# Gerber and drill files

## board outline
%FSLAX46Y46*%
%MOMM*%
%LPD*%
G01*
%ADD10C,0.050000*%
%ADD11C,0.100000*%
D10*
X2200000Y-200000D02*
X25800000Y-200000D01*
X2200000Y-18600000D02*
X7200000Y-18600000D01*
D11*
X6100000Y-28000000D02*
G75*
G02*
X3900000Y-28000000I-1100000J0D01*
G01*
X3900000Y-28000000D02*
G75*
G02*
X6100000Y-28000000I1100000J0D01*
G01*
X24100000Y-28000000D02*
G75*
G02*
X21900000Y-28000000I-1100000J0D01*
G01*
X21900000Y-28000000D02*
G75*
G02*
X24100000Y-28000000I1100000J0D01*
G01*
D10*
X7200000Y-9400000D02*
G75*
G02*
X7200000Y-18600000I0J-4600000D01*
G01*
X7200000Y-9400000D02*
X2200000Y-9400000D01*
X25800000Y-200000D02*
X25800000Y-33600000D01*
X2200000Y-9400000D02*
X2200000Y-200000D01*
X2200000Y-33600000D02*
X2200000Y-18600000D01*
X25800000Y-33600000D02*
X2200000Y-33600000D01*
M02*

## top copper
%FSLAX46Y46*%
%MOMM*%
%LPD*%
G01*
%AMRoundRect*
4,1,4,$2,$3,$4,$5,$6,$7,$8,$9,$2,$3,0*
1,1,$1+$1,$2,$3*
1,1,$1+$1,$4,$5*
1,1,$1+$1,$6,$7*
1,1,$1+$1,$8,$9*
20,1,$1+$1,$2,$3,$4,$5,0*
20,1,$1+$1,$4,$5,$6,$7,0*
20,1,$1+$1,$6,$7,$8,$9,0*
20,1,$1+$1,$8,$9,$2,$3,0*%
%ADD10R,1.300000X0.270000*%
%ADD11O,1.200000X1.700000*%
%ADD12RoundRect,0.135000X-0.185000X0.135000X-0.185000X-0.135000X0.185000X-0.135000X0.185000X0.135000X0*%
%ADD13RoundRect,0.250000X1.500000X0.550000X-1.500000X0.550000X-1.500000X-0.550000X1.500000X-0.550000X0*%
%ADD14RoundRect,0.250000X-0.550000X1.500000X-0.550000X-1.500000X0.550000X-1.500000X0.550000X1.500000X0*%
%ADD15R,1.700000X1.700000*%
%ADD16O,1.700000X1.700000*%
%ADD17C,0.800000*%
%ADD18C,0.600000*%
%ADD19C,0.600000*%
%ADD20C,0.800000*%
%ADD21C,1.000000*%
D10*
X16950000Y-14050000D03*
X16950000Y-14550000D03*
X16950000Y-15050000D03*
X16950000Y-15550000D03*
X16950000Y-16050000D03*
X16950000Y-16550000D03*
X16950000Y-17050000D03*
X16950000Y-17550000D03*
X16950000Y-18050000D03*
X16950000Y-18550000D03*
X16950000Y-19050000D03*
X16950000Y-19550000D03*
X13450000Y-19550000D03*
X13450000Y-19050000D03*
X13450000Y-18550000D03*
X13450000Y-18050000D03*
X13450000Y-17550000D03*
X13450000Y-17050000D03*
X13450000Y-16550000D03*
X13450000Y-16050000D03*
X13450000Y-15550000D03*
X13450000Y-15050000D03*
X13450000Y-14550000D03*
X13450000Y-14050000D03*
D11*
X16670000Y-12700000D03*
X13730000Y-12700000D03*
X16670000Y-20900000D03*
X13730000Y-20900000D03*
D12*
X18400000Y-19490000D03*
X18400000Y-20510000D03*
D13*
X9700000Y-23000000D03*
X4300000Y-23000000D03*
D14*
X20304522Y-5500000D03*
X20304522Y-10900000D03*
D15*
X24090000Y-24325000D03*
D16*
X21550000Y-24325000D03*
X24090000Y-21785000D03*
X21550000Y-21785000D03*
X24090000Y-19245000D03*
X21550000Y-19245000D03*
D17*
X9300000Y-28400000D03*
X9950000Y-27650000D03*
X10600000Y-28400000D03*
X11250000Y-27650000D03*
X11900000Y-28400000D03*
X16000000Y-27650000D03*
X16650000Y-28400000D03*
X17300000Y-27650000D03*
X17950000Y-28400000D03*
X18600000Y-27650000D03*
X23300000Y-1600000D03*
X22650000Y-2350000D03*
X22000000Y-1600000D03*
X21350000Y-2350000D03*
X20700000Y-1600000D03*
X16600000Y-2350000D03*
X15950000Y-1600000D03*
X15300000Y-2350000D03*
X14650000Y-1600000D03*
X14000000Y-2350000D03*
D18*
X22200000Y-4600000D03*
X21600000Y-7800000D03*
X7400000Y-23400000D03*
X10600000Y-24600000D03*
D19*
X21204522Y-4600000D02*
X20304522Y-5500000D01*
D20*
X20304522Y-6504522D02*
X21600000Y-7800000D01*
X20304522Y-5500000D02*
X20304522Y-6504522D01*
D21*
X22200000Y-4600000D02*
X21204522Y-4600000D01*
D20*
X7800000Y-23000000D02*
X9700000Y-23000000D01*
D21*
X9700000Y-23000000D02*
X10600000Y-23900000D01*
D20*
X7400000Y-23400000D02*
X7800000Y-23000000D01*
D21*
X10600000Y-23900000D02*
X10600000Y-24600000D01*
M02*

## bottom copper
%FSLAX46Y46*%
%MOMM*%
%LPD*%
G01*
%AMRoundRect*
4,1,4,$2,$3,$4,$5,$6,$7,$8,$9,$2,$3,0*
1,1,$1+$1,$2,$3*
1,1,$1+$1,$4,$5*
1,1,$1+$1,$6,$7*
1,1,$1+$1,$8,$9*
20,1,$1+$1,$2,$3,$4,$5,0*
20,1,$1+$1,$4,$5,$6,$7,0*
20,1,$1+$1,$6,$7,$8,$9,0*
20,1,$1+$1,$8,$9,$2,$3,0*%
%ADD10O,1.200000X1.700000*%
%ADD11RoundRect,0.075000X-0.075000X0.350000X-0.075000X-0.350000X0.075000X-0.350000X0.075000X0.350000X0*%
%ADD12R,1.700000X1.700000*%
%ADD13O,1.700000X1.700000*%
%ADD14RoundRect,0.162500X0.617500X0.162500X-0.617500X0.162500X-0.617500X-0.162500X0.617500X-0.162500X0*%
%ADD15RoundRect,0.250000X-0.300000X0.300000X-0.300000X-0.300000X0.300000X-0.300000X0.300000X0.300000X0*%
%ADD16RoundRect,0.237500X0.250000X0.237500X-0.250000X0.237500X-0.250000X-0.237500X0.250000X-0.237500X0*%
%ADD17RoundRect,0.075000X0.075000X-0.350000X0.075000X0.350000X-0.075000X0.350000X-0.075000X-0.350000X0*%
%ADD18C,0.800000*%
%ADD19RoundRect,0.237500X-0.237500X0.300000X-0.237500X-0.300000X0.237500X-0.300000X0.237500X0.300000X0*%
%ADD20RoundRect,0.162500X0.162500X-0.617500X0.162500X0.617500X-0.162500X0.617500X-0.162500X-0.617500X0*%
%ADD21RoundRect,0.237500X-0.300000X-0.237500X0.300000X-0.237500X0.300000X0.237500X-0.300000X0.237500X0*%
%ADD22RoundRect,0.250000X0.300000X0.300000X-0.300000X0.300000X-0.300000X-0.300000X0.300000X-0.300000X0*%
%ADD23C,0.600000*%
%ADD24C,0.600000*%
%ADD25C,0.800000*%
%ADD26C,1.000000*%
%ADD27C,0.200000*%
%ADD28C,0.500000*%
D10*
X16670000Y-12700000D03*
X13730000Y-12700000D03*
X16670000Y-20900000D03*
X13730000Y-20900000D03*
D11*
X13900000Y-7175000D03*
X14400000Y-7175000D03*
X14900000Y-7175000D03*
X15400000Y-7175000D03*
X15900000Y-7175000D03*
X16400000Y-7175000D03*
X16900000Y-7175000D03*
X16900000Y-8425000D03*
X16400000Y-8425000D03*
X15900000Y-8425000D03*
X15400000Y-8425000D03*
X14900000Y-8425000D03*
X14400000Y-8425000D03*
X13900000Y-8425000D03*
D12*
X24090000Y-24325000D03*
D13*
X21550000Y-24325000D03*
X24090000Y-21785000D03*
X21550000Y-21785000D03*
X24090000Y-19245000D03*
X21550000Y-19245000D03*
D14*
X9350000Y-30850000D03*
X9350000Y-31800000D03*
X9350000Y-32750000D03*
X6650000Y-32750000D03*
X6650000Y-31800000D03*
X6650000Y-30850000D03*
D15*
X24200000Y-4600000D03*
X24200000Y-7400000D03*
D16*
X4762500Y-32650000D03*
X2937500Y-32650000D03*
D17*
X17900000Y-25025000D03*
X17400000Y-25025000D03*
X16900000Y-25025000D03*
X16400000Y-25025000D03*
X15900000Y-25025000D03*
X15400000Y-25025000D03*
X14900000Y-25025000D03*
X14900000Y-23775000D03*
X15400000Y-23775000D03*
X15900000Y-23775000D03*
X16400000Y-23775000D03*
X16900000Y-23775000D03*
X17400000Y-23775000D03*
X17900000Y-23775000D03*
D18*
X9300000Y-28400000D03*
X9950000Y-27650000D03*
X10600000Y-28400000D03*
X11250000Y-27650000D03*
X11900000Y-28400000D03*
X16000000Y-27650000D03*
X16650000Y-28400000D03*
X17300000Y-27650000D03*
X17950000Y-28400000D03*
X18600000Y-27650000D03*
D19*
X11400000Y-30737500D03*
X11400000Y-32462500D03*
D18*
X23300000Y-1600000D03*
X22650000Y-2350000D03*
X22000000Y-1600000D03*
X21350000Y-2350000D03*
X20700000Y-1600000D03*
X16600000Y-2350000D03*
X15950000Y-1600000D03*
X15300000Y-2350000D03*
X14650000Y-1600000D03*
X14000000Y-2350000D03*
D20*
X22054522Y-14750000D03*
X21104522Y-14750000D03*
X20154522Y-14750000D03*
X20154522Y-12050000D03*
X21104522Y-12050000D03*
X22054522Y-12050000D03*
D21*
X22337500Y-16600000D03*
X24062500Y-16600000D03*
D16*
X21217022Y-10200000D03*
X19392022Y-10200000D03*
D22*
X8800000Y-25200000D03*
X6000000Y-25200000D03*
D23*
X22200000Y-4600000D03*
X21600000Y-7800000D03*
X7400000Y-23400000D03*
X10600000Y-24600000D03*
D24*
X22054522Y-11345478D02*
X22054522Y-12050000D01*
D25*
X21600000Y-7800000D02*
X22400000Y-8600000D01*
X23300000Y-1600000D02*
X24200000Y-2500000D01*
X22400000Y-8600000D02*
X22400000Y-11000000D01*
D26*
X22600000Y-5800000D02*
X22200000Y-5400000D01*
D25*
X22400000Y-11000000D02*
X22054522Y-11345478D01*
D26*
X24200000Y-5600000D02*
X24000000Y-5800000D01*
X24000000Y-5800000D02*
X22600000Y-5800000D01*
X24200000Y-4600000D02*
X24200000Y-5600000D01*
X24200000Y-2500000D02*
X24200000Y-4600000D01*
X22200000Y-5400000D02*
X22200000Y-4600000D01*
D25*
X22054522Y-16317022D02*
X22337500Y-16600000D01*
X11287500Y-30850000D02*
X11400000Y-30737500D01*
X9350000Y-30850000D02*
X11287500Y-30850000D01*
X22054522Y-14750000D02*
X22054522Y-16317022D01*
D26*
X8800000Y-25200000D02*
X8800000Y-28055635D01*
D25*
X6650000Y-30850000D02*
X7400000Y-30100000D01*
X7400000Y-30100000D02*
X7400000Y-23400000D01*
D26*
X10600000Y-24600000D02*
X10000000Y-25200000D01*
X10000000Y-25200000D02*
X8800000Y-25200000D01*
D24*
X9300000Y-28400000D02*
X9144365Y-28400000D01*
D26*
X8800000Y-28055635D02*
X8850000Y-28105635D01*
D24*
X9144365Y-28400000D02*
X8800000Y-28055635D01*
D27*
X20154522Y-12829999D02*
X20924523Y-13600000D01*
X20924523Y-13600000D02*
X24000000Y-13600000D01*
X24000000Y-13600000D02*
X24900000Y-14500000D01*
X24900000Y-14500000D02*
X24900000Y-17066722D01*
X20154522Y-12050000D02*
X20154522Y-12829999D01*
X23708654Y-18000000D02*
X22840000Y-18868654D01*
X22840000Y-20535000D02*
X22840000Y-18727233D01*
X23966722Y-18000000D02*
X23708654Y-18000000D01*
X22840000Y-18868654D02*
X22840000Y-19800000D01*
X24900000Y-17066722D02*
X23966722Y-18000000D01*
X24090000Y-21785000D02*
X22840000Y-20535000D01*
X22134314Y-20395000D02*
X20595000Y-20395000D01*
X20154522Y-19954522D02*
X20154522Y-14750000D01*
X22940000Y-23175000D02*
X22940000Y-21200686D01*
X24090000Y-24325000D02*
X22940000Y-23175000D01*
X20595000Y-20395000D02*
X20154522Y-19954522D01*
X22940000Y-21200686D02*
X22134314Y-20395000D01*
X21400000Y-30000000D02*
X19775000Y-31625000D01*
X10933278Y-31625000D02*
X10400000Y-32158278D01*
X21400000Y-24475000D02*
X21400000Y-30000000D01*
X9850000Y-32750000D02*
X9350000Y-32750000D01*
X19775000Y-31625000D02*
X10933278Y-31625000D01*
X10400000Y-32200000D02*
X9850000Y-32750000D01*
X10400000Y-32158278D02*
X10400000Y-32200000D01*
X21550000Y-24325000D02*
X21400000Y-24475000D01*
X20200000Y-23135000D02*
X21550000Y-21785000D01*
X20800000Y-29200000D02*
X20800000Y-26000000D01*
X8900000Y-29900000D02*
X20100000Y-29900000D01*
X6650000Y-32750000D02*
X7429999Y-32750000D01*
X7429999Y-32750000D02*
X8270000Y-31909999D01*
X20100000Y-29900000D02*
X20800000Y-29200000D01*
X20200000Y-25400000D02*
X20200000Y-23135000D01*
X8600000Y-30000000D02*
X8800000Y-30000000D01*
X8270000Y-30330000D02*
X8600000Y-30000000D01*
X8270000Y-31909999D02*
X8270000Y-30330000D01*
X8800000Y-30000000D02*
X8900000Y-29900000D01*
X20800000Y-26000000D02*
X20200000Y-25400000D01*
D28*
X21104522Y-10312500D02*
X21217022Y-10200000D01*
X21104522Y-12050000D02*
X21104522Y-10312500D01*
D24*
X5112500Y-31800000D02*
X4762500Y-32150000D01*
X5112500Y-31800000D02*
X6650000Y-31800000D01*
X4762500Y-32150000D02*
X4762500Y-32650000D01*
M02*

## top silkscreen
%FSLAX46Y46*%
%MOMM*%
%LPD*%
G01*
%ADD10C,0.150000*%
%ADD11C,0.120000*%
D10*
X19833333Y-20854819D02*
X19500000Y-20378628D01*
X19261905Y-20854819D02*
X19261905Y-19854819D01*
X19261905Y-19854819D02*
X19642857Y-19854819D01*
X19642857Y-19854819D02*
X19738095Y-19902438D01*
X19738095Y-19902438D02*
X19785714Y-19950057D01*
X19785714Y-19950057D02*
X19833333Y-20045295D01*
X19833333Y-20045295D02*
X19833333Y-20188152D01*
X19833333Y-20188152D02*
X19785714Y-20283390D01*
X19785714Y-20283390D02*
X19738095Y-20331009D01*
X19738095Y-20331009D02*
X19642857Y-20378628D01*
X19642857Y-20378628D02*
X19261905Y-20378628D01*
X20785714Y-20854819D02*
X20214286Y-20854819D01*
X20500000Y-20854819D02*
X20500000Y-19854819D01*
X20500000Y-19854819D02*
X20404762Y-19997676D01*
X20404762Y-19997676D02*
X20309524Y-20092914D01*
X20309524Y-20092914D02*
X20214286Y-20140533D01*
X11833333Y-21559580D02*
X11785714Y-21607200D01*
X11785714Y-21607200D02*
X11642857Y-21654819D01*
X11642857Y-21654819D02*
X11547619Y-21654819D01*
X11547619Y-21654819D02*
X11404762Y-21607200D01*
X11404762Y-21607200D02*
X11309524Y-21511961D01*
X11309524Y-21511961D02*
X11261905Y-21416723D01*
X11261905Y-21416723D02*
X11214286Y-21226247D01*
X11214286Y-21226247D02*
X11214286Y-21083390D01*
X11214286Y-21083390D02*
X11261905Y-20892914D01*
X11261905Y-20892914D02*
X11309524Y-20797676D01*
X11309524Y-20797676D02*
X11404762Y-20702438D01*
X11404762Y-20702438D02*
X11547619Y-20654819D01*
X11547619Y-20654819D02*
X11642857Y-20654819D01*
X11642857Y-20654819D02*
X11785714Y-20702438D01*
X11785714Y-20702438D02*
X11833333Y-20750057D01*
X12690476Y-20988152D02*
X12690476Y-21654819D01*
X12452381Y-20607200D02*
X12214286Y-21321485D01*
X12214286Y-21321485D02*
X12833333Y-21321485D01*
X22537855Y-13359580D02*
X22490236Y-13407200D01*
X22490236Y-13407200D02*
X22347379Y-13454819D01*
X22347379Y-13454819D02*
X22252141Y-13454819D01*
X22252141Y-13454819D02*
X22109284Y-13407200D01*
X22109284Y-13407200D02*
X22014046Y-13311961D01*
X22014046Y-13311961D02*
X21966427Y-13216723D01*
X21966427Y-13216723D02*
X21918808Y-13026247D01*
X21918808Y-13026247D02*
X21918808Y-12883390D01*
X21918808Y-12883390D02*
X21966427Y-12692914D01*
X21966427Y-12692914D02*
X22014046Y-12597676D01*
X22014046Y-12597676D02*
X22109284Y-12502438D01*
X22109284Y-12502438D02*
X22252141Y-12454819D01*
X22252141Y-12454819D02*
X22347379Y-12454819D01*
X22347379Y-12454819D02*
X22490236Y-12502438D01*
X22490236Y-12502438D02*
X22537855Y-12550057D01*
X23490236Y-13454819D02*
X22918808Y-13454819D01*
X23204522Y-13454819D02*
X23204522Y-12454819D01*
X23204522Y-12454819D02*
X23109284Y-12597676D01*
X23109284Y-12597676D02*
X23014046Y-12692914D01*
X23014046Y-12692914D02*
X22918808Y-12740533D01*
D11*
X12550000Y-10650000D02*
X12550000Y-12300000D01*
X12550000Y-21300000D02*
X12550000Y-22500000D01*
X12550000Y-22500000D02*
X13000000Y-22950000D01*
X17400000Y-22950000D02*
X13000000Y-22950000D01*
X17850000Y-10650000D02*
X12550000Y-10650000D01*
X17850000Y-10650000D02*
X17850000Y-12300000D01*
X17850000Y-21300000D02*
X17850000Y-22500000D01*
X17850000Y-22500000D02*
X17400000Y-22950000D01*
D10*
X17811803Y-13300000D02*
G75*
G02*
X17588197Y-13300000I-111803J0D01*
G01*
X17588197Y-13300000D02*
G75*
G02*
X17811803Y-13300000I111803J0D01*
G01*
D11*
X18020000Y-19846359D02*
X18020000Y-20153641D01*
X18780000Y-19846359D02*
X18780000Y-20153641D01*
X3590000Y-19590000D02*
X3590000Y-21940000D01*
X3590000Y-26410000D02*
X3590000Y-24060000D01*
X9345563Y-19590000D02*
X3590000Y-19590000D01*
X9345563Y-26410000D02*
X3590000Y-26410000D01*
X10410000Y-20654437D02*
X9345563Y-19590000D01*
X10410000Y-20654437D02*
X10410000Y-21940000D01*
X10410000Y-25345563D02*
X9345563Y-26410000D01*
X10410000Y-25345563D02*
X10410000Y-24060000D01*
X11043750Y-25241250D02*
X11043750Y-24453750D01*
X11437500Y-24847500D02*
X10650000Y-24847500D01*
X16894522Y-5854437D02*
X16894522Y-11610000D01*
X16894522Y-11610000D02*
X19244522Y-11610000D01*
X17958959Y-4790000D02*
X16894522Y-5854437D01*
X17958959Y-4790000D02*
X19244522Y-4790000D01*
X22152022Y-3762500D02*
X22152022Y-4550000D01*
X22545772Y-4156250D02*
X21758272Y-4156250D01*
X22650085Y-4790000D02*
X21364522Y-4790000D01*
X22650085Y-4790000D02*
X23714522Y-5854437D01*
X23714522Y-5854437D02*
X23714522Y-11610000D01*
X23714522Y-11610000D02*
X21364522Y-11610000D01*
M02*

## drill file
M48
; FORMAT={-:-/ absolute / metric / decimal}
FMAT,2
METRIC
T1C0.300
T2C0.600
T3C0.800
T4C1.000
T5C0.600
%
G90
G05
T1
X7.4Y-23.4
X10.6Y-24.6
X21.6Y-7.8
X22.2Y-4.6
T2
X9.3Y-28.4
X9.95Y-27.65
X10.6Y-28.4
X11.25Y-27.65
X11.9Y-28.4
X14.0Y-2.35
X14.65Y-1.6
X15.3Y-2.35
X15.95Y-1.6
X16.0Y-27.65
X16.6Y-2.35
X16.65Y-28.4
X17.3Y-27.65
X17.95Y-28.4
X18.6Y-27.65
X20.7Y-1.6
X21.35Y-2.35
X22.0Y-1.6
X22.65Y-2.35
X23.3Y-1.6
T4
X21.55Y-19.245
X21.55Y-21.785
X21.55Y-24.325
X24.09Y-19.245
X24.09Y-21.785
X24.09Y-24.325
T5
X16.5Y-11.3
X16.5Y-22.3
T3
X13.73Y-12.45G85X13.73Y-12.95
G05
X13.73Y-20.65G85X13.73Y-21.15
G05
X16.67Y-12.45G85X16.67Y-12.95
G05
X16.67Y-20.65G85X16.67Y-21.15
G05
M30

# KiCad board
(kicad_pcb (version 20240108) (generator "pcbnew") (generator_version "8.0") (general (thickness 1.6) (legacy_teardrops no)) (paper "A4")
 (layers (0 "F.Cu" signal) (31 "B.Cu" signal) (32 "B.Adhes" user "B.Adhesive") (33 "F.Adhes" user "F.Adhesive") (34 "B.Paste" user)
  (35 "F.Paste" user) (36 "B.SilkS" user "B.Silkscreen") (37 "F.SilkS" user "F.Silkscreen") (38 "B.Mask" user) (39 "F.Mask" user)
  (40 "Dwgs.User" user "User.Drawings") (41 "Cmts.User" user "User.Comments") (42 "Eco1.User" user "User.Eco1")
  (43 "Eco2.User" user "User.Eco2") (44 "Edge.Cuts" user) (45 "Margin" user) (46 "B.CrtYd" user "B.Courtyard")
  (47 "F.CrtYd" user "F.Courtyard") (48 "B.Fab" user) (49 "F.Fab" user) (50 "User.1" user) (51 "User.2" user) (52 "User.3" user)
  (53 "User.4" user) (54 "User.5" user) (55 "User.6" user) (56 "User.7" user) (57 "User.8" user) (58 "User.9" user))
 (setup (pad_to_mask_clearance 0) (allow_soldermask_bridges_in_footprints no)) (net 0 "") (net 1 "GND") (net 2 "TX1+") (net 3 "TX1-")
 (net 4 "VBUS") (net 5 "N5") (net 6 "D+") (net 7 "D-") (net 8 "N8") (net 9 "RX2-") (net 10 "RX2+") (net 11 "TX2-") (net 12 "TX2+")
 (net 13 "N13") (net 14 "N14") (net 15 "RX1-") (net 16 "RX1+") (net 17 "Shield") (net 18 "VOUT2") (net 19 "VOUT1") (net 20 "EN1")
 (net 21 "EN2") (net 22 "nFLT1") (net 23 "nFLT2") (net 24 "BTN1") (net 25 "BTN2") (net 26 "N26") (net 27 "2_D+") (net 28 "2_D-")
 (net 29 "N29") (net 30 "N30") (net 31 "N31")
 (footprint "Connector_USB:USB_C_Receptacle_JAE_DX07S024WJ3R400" (layer "F.Cu") (at 15.2 16.8 -90)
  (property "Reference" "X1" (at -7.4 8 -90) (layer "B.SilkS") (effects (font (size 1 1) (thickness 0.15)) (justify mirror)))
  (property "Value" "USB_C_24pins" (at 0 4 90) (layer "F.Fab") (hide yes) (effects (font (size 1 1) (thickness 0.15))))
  (fp_line (start -6.15 2.65) (end -4.5 2.65) (stroke (width 0.12) (type solid)) (layer "F.SilkS"))
  (fp_line (start 4.5 2.65) (end 5.7 2.65) (stroke (width 0.12) (type solid)) (layer "F.SilkS"))
  (fp_line (start 5.7 2.65) (end 6.15 2.2) (stroke (width 0.12) (type solid)) (layer "F.SilkS"))
  (fp_line (start 6.15 -2.2) (end 6.15 2.2) (stroke (width 0.12) (type solid)) (layer "F.SilkS"))
  (fp_line (start -6.15 -2.65) (end -6.15 2.65) (stroke (width 0.12) (type solid)) (layer "F.SilkS"))
  (fp_line (start -6.15 -2.65) (end -4.5 -2.65) (stroke (width 0.12) (type solid)) (layer "F.SilkS"))
  (fp_line (start 4.5 -2.65) (end 5.7 -2.65) (stroke (width 0.12) (type solid)) (layer "F.SilkS"))
  (fp_line (start 5.7 -2.65) (end 6.15 -2.2) (stroke (width 0.12) (type solid)) (layer "F.SilkS"))
  (fp_circle (center -3.5 -2.5) (end -3.388197 -2.5) (stroke (width 0.15) (type solid)) (fill none) (layer "F.SilkS"))
  (pad "" np_thru_hole circle (at -5.5 -1.3 270) (size 0.6 0.6) (drill 0.6) (layers "*.Cu" "*.Mask"))
  (pad "" np_thru_hole circle (at 5.5 -1.3 270) (size 0.6 0.6) (drill 0.6) (layers "*.Cu" "*.Mask"))
  (pad "A1" smd rect (at -2.75 -1.75 270) (size 0.27 1.3) (layers "F.Cu" "F.Paste" "F.Mask") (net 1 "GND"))
  (pad "A2" smd rect (at -2.25 -1.75 270) (size 0.27 1.3) (layers "F.Cu" "F.Paste" "F.Mask") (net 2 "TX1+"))
  (pad "A3" smd rect (at -1.75 -1.75 270) (size 0.27 1.3) (layers "F.Cu" "F.Paste" "F.Mask") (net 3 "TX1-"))
  (pad "A4" smd rect (at -1.25 -1.75 270) (size 0.27 1.3) (layers "F.Cu" "F.Paste" "F.Mask") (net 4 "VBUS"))
  (pad "A5" smd rect (at -0.75 -1.75 270) (size 0.27 1.3) (layers "F.Cu" "F.Paste" "F.Mask") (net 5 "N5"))
  (pad "A6" smd rect (at -0.25 -1.75 270) (size 0.27 1.3) (layers "F.Cu" "F.Paste" "F.Mask") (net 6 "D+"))
  (pad "A7" smd rect (at 0.25 -1.75 270) (size 0.27 1.3) (layers "F.Cu" "F.Paste" "F.Mask") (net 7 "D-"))
  (pad "A8" smd rect (at 0.75 -1.75 270) (size 0.27 1.3) (layers "F.Cu" "F.Paste" "F.Mask") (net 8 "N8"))
  (pad "A9" smd rect (at 1.25 -1.75 270) (size 0.27 1.3) (layers "F.Cu" "F.Paste" "F.Mask") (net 4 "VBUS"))
  (pad "A10" smd rect (at 1.75 -1.75 270) (size 0.27 1.3) (layers "F.Cu" "F.Paste" "F.Mask") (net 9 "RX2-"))
  (pad "A11" smd rect (at 2.25 -1.75 270) (size 0.27 1.3) (layers "F.Cu" "F.Paste" "F.Mask") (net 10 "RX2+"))
  (pad "A12" smd rect (at 2.75 -1.75 270) (size 0.27 1.3) (layers "F.Cu" "F.Paste" "F.Mask") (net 1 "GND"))
  (pad "B1" smd rect (at 2.75 1.75 270) (size 0.27 1.3) (layers "F.Cu" "F.Paste" "F.Mask") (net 1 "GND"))
  (pad "B2" smd rect (at 2.25 1.75 270) (size 0.27 1.3) (layers "F.Cu" "F.Paste" "F.Mask") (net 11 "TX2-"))
  (pad "B3" smd rect (at 1.75 1.75 270) (size 0.27 1.3) (layers "F.Cu" "F.Paste" "F.Mask") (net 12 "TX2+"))
  (pad "B4" smd rect (at 1.25 1.75 270) (size 0.27 1.3) (layers "F.Cu" "F.Paste" "F.Mask") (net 4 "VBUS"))
  (pad "B5" smd rect (at 0.75 1.75 270) (size 0.27 1.3) (layers "F.Cu" "F.Paste" "F.Mask") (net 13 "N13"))
  (pad "B6" smd rect (at 0.25 1.75 270) (size 0.27 1.3) (layers "F.Cu" "F.Paste" "F.Mask") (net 6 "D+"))
  (pad "B7" smd rect (at -0.25 1.75 270) (size 0.27 1.3) (layers "F.Cu" "F.Paste" "F.Mask") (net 7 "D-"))
  (pad "B8" smd rect (at -0.75 1.75 270) (size 0.27 1.3) (layers "F.Cu" "F.Paste" "F.Mask") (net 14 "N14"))
  (pad "B9" smd rect (at -1.25 1.75 270) (size 0.27 1.3) (layers "F.Cu" "F.Paste" "F.Mask") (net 4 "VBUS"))
  (pad "B10" smd rect (at -1.75 1.75 270) (size 0.27 1.3) (layers "F.Cu" "F.Paste" "F.Mask") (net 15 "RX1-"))
  (pad "B11" smd rect (at -2.25 1.75 270) (size 0.27 1.3) (layers "F.Cu" "F.Paste" "F.Mask") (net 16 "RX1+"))
  (pad "B12" smd rect (at -2.75 1.75 270) (size 0.27 1.3) (layers "F.Cu" "F.Paste" "F.Mask") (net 1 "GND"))
  (pad "S1" thru_hole oval (at -4.1 -1.47) (size 1.2 1.7) (drill oval 0.8 1.3) (layers "*.Cu" "*.Mask") (remove_unused_layers no)
   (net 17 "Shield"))
  (pad "S1" thru_hole oval (at -4.1 1.47) (size 1.2 1.7) (drill oval 0.8 1.3) (layers "*.Cu" "*.Mask") (remove_unused_layers no)
   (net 17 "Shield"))
  (pad "S1" thru_hole oval (at 4.1 -1.47) (size 1.2 1.7) (drill oval 0.8 1.3) (layers "*.Cu" "*.Mask") (remove_unused_layers no)
   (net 17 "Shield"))
  (pad "S1" thru_hole oval (at 4.1 1.47) (size 1.2 1.7) (drill oval 0.8 1.3) (layers "*.Cu" "*.Mask") (remove_unused_layers no)
   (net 17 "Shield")))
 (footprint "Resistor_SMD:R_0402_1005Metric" (layer "F.Cu") (at 18.4 20 -90)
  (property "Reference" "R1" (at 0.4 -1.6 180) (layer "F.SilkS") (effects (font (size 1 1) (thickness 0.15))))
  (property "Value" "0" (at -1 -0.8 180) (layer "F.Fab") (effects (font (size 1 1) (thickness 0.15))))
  (fp_line (start -0.153641 0.38) (end 0.153641 0.38) (stroke (width 0.12) (type solid)) (layer "F.SilkS"))
  (fp_line (start -0.153641 -0.38) (end 0.153641 -0.38) (stroke (width 0.12) (type solid)) (layer "F.SilkS"))
  (pad "1" smd roundrect (at -0.51 0 270) (size 0.54 0.64) (layers "F.Cu" "F.Paste" "F.Mask") (roundrect_rratio 0.25) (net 17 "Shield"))
  (pad "2" smd roundrect (at 0.51 0 270) (size 0.54 0.64) (layers "F.Cu" "F.Paste" "F.Mask") (roundrect_rratio 0.25) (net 1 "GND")))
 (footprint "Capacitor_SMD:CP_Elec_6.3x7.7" (layer "F.Cu") (at 7 23 180)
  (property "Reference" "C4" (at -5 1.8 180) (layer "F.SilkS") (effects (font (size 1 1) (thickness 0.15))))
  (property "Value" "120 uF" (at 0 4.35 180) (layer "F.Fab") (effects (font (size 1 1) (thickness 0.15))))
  (fp_line (start 3.41 3.41) (end 3.41 1.06) (stroke (width 0.12) (type solid)) (layer "F.SilkS"))
  (fp_line (start 3.41 -3.41) (end 3.41 -1.06) (stroke (width 0.12) (type solid)) (layer "F.SilkS"))
  (fp_line (start -2.345563 3.41) (end 3.41 3.41) (stroke (width 0.12) (type solid)) (layer "F.SilkS"))
  (fp_line (start -2.345563 -3.41) (end 3.41 -3.41) (stroke (width 0.12) (type solid)) (layer "F.SilkS"))
  (fp_line (start -3.41 2.345563) (end -2.345563 3.41) (stroke (width 0.12) (type solid)) (layer "F.SilkS"))
  (fp_line (start -3.41 2.345563) (end -3.41 1.06) (stroke (width 0.12) (type solid)) (layer "F.SilkS"))
  (fp_line (start -3.41 -2.345563) (end -2.345563 -3.41) (stroke (width 0.12) (type solid)) (layer "F.SilkS"))
  (fp_line (start -3.41 -2.345563) (end -3.41 -1.06) (stroke (width 0.12) (type solid)) (layer "F.SilkS"))
  (fp_line (start -4.04375 -2.24125) (end -4.04375 -1.45375) (stroke (width 0.12) (type solid)) (layer "F.SilkS"))
  (fp_line (start -4.4375 -1.8475) (end -3.65 -1.8475) (stroke (width 0.12) (type solid)) (layer "F.SilkS"))
  (pad "1" smd roundrect (at -2.7 0 180) (size 3.5 1.6) (layers "F.Cu" "F.Paste" "F.Mask") (roundrect_rratio 0.15625) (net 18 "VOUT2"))
  (pad "2" smd roundrect (at 2.7 0 180) (size 3.5 1.6) (layers "F.Cu" "F.Paste" "F.Mask") (roundrect_rratio 0.15625) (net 1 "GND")))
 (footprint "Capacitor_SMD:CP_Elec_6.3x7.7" (layer "F.Cu") (at 20.304522 8.2 -90)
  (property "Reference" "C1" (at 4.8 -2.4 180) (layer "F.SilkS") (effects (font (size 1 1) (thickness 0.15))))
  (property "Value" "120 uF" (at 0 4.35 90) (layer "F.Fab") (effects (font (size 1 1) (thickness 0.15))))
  (fp_line (start -2.345563 3.41) (end 3.41 3.41) (stroke (width 0.12) (type solid)) (layer "F.SilkS"))
  (fp_line (start 3.41 3.41) (end 3.41 1.06) (stroke (width 0.12) (type solid)) (layer "F.SilkS"))
  (fp_line (start -3.41 2.345563) (end -2.345563 3.41) (stroke (width 0.12) (type solid)) (layer "F.SilkS"))
  (fp_line (start -3.41 2.345563) (end -3.41 1.06) (stroke (width 0.12) (type solid)) (layer "F.SilkS"))
  (fp_line (start -4.4375 -1.8475) (end -3.65 -1.8475) (stroke (width 0.12) (type solid)) (layer "F.SilkS"))
  (fp_line (start -4.04375 -2.24125) (end -4.04375 -1.45375) (stroke (width 0.12) (type solid)) (layer "F.SilkS"))
  (fp_line (start -3.41 -2.345563) (end -3.41 -1.06) (stroke (width 0.12) (type solid)) (layer "F.SilkS"))
  (fp_line (start -3.41 -2.345563) (end -2.345563 -3.41) (stroke (width 0.12) (type solid)) (layer "F.SilkS"))
  (fp_line (start -2.345563 -3.41) (end 3.41 -3.41) (stroke (width 0.12) (type solid)) (layer "F.SilkS"))
  (fp_line (start 3.41 -3.41) (end 3.41 -1.06) (stroke (width 0.12) (type solid)) (layer "F.SilkS"))
  (pad "1" smd roundrect (at -2.7 0 270) (size 3.5 1.6) (layers "F.Cu" "F.Paste" "F.Mask") (roundrect_rratio 0.15625) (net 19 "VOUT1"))
  (pad "2" smd roundrect (at 2.7 0 270) (size 3.5 1.6) (layers "F.Cu" "F.Paste" "F.Mask") (roundrect_rratio 0.15625) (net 1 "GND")))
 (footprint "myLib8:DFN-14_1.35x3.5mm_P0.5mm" (layer "B.Cu") (at 15.4 7.8 -90)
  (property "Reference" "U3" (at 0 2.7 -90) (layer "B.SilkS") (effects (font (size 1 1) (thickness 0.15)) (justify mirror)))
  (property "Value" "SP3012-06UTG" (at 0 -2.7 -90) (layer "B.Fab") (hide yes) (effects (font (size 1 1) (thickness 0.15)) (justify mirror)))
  (pad "1" smd roundrect (at -0.625 1.5 270) (size 0.85 0.3) (layers "B.Cu" "B.Paste" "B.Mask") (roundrect_rratio 0.25) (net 16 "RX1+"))
  (pad "2" smd roundrect (at -0.625 1 270) (size 0.85 0.3) (layers "B.Cu" "B.Paste" "B.Mask") (roundrect_rratio 0.25) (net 15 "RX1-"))
  (pad "3" smd roundrect (at -0.625 0.5 270) (size 0.85 0.3) (layers "B.Cu" "B.Paste" "B.Mask") (roundrect_rratio 0.25) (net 2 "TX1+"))
  (pad "4" smd roundrect (at -0.625 0 270) (size 0.85 0.3) (layers "B.Cu" "B.Paste" "B.Mask") (roundrect_rratio 0.25) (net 3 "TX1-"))
  (pad "5" smd roundrect (at -0.625 -0.5 270) (size 0.85 0.3) (layers "B.Cu" "B.Paste" "B.Mask") (roundrect_rratio 0.25) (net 1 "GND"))
  (pad "6" smd roundrect (at -0.625 -1 270) (size 0.85 0.3) (layers "B.Cu" "B.Paste" "B.Mask") (roundrect_rratio 0.25) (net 6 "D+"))
  (pad "7" smd roundrect (at -0.625 -1.5 270) (size 0.85 0.3) (layers "B.Cu" "B.Paste" "B.Mask") (roundrect_rratio 0.25) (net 7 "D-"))
  (pad "8" smd roundrect (at 0.625 -1.5 270) (size 0.85 0.3) (layers "B.Cu" "B.Paste" "B.Mask") (roundrect_rratio 0.25) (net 7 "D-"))
  (pad "9" smd roundrect (at 0.625 -1 270) (size 0.85 0.3) (layers "B.Cu" "B.Paste" "B.Mask") (roundrect_rratio 0.25) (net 6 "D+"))
  (pad "10" smd roundrect (at 0.625 -0.5 270) (size 0.85 0.3) (layers "B.Cu" "B.Paste" "B.Mask") (roundrect_rratio 0.25) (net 1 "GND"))
  (pad "11" smd roundrect (at 0.625 0 270) (size 0.85 0.3) (layers "B.Cu" "B.Paste" "B.Mask") (roundrect_rratio 0.25) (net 3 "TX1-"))
  (pad "12" smd roundrect (at 0.625 0.5 270) (size 0.85 0.3) (layers "B.Cu" "B.Paste" "B.Mask") (roundrect_rratio 0.25) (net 2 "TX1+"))
  (pad "13" smd roundrect (at 0.625 1 270) (size 0.85 0.3) (layers "B.Cu" "B.Paste" "B.Mask") (roundrect_rratio 0.25) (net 15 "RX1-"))
  (pad "14" smd roundrect (at 0.625 1.5 270) (size 0.85 0.3) (layers "B.Cu" "B.Paste" "B.Mask") (roundrect_rratio 0.25) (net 16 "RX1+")))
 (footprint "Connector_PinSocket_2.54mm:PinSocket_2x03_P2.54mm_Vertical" (layer "B.Cu") (at 24.09 24.325)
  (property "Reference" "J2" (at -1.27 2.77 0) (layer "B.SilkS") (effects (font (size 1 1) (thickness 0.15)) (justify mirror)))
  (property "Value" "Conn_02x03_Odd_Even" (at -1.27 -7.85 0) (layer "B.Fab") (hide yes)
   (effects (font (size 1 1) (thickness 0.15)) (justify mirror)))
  (pad "1" thru_hole rect (at 0 0) (size 1.7 1.7) (drill 1) (layers "*.Cu" "*.Mask") (remove_unused_layers no) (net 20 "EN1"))
  (pad "2" thru_hole oval (at -2.54 0) (size 1.7 1.7) (drill 1) (layers "*.Cu" "*.Mask") (remove_unused_layers no) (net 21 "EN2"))
  (pad "3" thru_hole oval (at 0 -2.54) (size 1.7 1.7) (drill 1) (layers "*.Cu" "*.Mask") (remove_unused_layers no) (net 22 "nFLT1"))
  (pad "4" thru_hole oval (at -2.54 -2.54) (size 1.7 1.7) (drill 1) (layers "*.Cu" "*.Mask") (remove_unused_layers no) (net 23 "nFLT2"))
  (pad "5" thru_hole oval (at 0 -5.08) (size 1.7 1.7) (drill 1) (layers "*.Cu" "*.Mask") (remove_unused_layers no) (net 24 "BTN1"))
  (pad "6" thru_hole oval (at -2.54 -5.08) (size 1.7 1.7) (drill 1) (layers "*.Cu" "*.Mask") (remove_unused_layers no) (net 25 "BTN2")))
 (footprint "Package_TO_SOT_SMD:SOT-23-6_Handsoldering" (layer "B.Cu") (at 8 31.8 180)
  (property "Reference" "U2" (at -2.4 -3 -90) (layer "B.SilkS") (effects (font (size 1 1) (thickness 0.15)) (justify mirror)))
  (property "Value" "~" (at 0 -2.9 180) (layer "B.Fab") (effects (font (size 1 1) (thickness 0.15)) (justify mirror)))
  (pad "1" smd roundrect (at -1.35 0.95 180) (size 1.56 0.65) (layers "B.Cu" "B.Paste" "B.Mask") (roundrect_rratio 0.25) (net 4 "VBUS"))
  (pad "2" smd roundrect (at -1.35 0 180) (size 1.56 0.65) (layers "B.Cu" "B.Paste" "B.Mask") (roundrect_rratio 0.25) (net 1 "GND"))
  (pad "3" smd roundrect (at -1.35 -0.95 180) (size 1.56 0.65) (layers "B.Cu" "B.Paste" "B.Mask") (roundrect_rratio 0.25) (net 21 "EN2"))
  (pad "4" smd roundrect (at 1.35 -0.95 180) (size 1.56 0.65) (layers "B.Cu" "B.Paste" "B.Mask") (roundrect_rratio 0.25) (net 23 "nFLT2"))
  (pad "5" smd roundrect (at 1.35 0 180) (size 1.56 0.65) (layers "B.Cu" "B.Paste" "B.Mask") (roundrect_rratio 0.25) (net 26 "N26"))
  (pad "6" smd roundrect (at 1.35 0.95 180) (size 1.56 0.65) (layers "B.Cu" "B.Paste" "B.Mask") (roundrect_rratio 0.25) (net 18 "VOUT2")))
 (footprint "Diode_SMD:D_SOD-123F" (layer "B.Cu") (at 24.2 6 -90)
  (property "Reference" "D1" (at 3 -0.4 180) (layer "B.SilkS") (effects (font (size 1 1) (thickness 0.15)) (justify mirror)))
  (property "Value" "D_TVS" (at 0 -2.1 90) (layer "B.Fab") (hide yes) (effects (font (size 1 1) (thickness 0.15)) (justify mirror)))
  (pad "1" smd roundrect (at -1.4 0 270) (size 1.1 1.1) (layers "B.Cu" "B.Paste" "B.Mask") (roundrect_rratio 0.2272727273) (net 19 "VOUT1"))
  (pad "2" smd roundrect (at 1.4 0 270) (size 1.1 1.1) (layers "B.Cu" "B.Paste" "B.Mask") (roundrect_rratio 0.2272727273) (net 1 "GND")))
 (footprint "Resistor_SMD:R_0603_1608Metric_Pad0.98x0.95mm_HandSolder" (layer "B.Cu") (at 3.85 32.65 180)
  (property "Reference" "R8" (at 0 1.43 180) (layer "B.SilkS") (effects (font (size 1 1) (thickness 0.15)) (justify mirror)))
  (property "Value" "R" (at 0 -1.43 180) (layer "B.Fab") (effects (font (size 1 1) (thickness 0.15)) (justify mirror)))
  (pad "1" smd roundrect (at -0.9125 0 180) (size 0.975 0.95) (layers "B.Cu" "B.Paste" "B.Mask") (roundrect_rratio 0.25) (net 26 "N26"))
  (pad "2" smd roundrect (at 0.9125 0 180) (size 0.975 0.95) (layers "B.Cu" "B.Paste" "B.Mask") (roundrect_rratio 0.25) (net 1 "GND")))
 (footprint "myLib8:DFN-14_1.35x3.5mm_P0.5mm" (layer "B.Cu") (at 16.4 24.4 90)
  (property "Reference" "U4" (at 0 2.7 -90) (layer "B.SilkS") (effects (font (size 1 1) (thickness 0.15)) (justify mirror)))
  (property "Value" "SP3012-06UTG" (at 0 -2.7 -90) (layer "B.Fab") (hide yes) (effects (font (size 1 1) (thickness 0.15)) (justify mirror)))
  (pad "1" smd roundrect (at -0.625 1.5 90) (size 0.85 0.3) (layers "B.Cu" "B.Paste" "B.Mask") (roundrect_rratio 0.25) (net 10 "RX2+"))
  (pad "2" smd roundrect (at -0.625 1 90) (size 0.85 0.3) (layers "B.Cu" "B.Paste" "B.Mask") (roundrect_rratio 0.25) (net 9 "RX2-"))
  (pad "3" smd roundrect (at -0.625 0.5 90) (size 0.85 0.3) (layers "B.Cu" "B.Paste" "B.Mask") (roundrect_rratio 0.25) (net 11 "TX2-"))
  (pad "4" smd roundrect (at -0.625 0 90) (size 0.85 0.3) (layers "B.Cu" "B.Paste" "B.Mask") (roundrect_rratio 0.25) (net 12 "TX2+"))
  (pad "5" smd roundrect (at -0.625 -0.5 90) (size 0.85 0.3) (layers "B.Cu" "B.Paste" "B.Mask") (roundrect_rratio 0.25) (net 1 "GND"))
  (pad "6" smd roundrect (at -0.625 -1 90) (size 0.85 0.3) (layers "B.Cu" "B.Paste" "B.Mask") (roundrect_rratio 0.25) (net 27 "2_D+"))
  (pad "7" smd roundrect (at -0.625 -1.5 90) (size 0.85 0.3) (layers "B.Cu" "B.Paste" "B.Mask") (roundrect_rratio 0.25) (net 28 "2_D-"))
  (pad "8" smd roundrect (at 0.625 -1.5 90) (size 0.85 0.3) (layers "B.Cu" "B.Paste" "B.Mask") (roundrect_rratio 0.25) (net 28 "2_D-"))
  (pad "9" smd roundrect (at 0.625 -1 90) (size 0.85 0.3) (layers "B.Cu" "B.Paste" "B.Mask") (roundrect_rratio 0.25) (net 27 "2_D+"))
  (pad "10" smd roundrect (at 0.625 -0.5 90) (size 0.85 0.3) (layers "B.Cu" "B.Paste" "B.Mask") (roundrect_rratio 0.25) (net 1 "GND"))
  (pad "11" smd roundrect (at 0.625 0 90) (size 0.85 0.3) (layers "B.Cu" "B.Paste" "B.Mask") (roundrect_rratio 0.25) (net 12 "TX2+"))
  (pad "12" smd roundrect (at 0.625 0.5 90) (size 0.85 0.3) (layers "B.Cu" "B.Paste" "B.Mask") (roundrect_rratio 0.25) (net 11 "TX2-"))
  (pad "13" smd roundrect (at 0.625 1 90) (size 0.85 0.3) (layers "B.Cu" "B.Paste" "B.Mask") (roundrect_rratio 0.25) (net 9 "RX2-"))
  (pad "14" smd roundrect (at 0.625 1.5 90) (size 0.85 0.3) (layers "B.Cu" "B.Paste" "B.Mask") (roundrect_rratio 0.25) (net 10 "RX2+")))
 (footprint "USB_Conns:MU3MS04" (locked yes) (layer "B.Cu") (at 9.3 28.4 180)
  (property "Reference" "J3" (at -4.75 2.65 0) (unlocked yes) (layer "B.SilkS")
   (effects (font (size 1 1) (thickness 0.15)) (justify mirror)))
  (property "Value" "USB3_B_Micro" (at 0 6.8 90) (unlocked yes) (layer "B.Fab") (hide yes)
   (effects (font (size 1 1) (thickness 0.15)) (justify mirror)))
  (pad "1" thru_hole circle (at 0 0 180) (size 0.8 0.8) (drill 0.6) (layers "*.Cu" "*.Mask") (remove_unused_layers no) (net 18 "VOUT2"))
  (pad "2" thru_hole circle (at -0.65 0.75 180) (size 0.8 0.8) (drill 0.6) (layers "*.Cu" "*.Mask") (remove_unused_layers no)
   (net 28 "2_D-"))
  (pad "3" thru_hole circle (at -1.3 0 180) (size 0.8 0.8) (drill 0.6) (layers "*.Cu" "*.Mask") (remove_unused_layers no) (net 27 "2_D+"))
  (pad "4" thru_hole circle (at -1.95 0.75 180) (size 0.8 0.8) (drill 0.6) (layers "*.Cu" "*.Mask") (remove_unused_layers no) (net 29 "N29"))
  (pad "5" thru_hole circle (at -2.6 0 180) (size 0.8 0.8) (drill 0.6) (layers "*.Cu" "*.Mask") (remove_unused_layers no) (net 1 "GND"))
  (pad "6" thru_hole circle (at -6.7 0.75 180) (size 0.8 0.8) (drill 0.6) (layers "*.Cu" "*.Mask") (remove_unused_layers no) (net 12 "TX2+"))
  (pad "7" thru_hole circle (at -7.35 0 180) (size 0.8 0.8) (drill 0.6) (layers "*.Cu" "*.Mask") (remove_unused_layers no) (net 11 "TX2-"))
  (pad "8" thru_hole circle (at -8 0.75 180) (size 0.8 0.8) (drill 0.6) (layers "*.Cu" "*.Mask") (remove_unused_layers no) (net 1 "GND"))
  (pad "9" thru_hole circle (at -8.65 0 180) (size 0.8 0.8) (drill 0.6) (layers "*.Cu" "*.Mask") (remove_unused_layers no) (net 9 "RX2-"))
  (pad "10" thru_hole circle (at -9.3 0.75 180) (size 0.8 0.8) (drill 0.6) (layers "*.Cu" "*.Mask") (remove_unused_layers no)
   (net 10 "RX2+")))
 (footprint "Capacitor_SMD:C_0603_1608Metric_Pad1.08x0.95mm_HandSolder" (layer "B.Cu") (at 11.4 31.6 -90)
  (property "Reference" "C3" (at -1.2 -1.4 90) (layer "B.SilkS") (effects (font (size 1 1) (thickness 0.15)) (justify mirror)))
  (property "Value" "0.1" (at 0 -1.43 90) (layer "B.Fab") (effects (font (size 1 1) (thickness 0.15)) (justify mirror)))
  (pad "1" smd roundrect (at -0.8625 0 270) (size 1.075 0.95) (layers "B.Cu" "B.Paste" "B.Mask") (roundrect_rratio 0.25) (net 4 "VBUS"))
  (pad "2" smd roundrect (at 0.8625 0 270) (size 1.075 0.95) (layers "B.Cu" "B.Paste" "B.Mask") (roundrect_rratio 0.25) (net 1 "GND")))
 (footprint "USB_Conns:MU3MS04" (layer "B.Cu") (at 23.3 1.6)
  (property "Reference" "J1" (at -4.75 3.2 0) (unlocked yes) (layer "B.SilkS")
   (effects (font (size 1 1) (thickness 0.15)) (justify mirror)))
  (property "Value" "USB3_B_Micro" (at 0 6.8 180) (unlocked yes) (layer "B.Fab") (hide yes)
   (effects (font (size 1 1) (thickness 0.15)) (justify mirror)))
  (pad "1" thru_hole circle (at 0 0) (size 0.8 0.8) (drill 0.6) (layers "*.Cu" "*.Mask") (remove_unused_layers no) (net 19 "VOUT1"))
  (pad "2" thru_hole circle (at -0.65 0.75) (size 0.8 0.8) (drill 0.6) (layers "*.Cu" "*.Mask") (remove_unused_layers no) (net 7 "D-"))
  (pad "3" thru_hole circle (at -1.3 0) (size 0.8 0.8) (drill 0.6) (layers "*.Cu" "*.Mask") (remove_unused_layers no) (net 6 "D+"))
  (pad "4" thru_hole circle (at -1.95 0.75) (size 0.8 0.8) (drill 0.6) (layers "*.Cu" "*.Mask") (remove_unused_layers no) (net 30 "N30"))
  (pad "5" thru_hole circle (at -2.6 0) (size 0.8 0.8) (drill 0.6) (layers "*.Cu" "*.Mask") (remove_unused_layers no) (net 1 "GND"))
  (pad "6" thru_hole circle (at -6.7 0.75) (size 0.8 0.8) (drill 0.6) (layers "*.Cu" "*.Mask") (remove_unused_layers no) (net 3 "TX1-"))
  (pad "7" thru_hole circle (at -7.35 0) (size 0.8 0.8) (drill 0.6) (layers "*.Cu" "*.Mask") (remove_unused_layers no) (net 2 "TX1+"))
  (pad "8" thru_hole circle (at -8 0.75) (size 0.8 0.8) (drill 0.6) (layers "*.Cu" "*.Mask") (remove_unused_layers no) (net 1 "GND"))
  (pad "9" thru_hole circle (at -8.65 0) (size 0.8 0.8) (drill 0.6) (layers "*.Cu" "*.Mask") (remove_unused_layers no) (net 15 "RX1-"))
  (pad "10" thru_hole circle (at -9.3 0.75) (size 0.8 0.8) (drill 0.6) (layers "*.Cu" "*.Mask") (remove_unused_layers no) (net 16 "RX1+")))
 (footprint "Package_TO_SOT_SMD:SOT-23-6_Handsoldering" (layer "B.Cu") (at 21.104522 13.4 90)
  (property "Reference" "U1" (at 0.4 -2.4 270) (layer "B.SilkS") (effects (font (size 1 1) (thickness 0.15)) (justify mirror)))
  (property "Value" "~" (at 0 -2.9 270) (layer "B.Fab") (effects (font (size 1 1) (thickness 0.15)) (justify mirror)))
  (pad "1" smd roundrect (at -1.35 0.95 90) (size 1.56 0.65) (layers "B.Cu" "B.Paste" "B.Mask") (roundrect_rratio 0.25) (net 4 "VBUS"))
  (pad "2" smd roundrect (at -1.35 0 90) (size 1.56 0.65) (layers "B.Cu" "B.Paste" "B.Mask") (roundrect_rratio 0.25) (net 1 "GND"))
  (pad "3" smd roundrect (at -1.35 -0.95 90) (size 1.56 0.65) (layers "B.Cu" "B.Paste" "B.Mask") (roundrect_rratio 0.25) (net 20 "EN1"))
  (pad "4" smd roundrect (at 1.35 -0.95 90) (size 1.56 0.65) (layers "B.Cu" "B.Paste" "B.Mask") (roundrect_rratio 0.25) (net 22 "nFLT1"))
  (pad "5" smd roundrect (at 1.35 0 90) (size 1.56 0.65) (layers "B.Cu" "B.Paste" "B.Mask") (roundrect_rratio 0.25) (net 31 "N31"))
  (pad "6" smd roundrect (at 1.35 0.95 90) (size 1.56 0.65) (layers "B.Cu" "B.Paste" "B.Mask") (roundrect_rratio 0.25) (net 19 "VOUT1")))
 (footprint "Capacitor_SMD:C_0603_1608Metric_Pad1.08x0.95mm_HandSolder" (layer "B.Cu") (at 23.2 16.6)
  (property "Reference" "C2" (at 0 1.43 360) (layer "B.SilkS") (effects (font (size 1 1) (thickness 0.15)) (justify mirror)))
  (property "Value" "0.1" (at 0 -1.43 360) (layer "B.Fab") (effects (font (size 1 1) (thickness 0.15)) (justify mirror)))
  (pad "1" smd roundrect (at -0.8625 0) (size 1.075 0.95) (layers "B.Cu" "B.Paste" "B.Mask") (roundrect_rratio 0.25) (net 4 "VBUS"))
  (pad "2" smd roundrect (at 0.8625 0) (size 1.075 0.95) (layers "B.Cu" "B.Paste" "B.Mask") (roundrect_rratio 0.25) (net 1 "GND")))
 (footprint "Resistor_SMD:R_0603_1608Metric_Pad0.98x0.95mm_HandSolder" (layer "B.Cu") (at 20.304522 10.2 180)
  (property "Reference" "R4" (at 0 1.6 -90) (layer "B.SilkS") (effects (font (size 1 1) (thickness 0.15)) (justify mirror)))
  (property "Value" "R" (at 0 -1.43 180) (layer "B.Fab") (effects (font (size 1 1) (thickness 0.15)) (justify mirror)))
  (pad "1" smd roundrect (at -0.9125 0 180) (size 0.975 0.95) (layers "B.Cu" "B.Paste" "B.Mask") (roundrect_rratio 0.25) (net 31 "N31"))
  (pad "2" smd roundrect (at 0.9125 0 180) (size 0.975 0.95) (layers "B.Cu" "B.Paste" "B.Mask") (roundrect_rratio 0.25) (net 1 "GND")))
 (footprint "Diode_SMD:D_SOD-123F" (layer "B.Cu") (at 7.4 25.2 180)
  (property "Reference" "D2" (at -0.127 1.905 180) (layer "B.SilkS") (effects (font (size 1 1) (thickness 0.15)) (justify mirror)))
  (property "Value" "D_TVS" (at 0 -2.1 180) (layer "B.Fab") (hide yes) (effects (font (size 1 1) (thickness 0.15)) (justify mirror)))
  (pad "1" smd roundrect (at -1.4 0 180) (size 1.1 1.1) (layers "B.Cu" "B.Paste" "B.Mask") (roundrect_rratio 0.2272727273) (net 18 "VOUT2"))
  (pad "2" smd roundrect (at 1.4 0 180) (size 1.1 1.1) (layers "B.Cu" "B.Paste" "B.Mask") (roundrect_rratio 0.2272727273) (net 1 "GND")))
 (gr_line (start 2.2 0.2) (end 25.8 0.2) (locked yes) (stroke (width 0.05) (type default)) (layer "Edge.Cuts"))
 (gr_line (start 2.2 18.6) (end 7.2 18.6) (locked yes) (stroke (width 0.05) (type default)) (layer "Edge.Cuts"))
 (gr_circle (center 5 28) (end 6.1 28) (locked yes) (stroke (width 0.1) (type default)) (fill none) (layer "Edge.Cuts"))
 (gr_circle (center 23 28) (end 24.1 28) (locked yes) (stroke (width 0.1) (type default)) (fill none) (layer "Edge.Cuts"))
 (gr_arc (start 7.2 9.4) (mid 11.8 14) (end 7.2 18.6) (locked yes) (stroke (width 0.05) (type default)) (layer "Edge.Cuts"))
 (gr_line (start 7.2 9.4) (end 2.2 9.4) (locked yes) (stroke (width 0.05) (type default)) (layer "Edge.Cuts"))
 (gr_line (start 25.8 0.2) (end 25.8 33.6) (locked yes) (stroke (width 0.05) (type default)) (layer "Edge.Cuts"))
 (gr_line (start 2.2 9.4) (end 2.2 0.2) (locked yes) (stroke (width 0.05) (type default)) (layer "Edge.Cuts"))
 (gr_line (start 2.2 33.6) (end 2.2 18.6) (locked yes) (stroke (width 0.05) (type default)) (layer "Edge.Cuts"))
 (gr_line (start 25.8 33.6) (end 2.2 33.6) (locked yes) (stroke (width 0.05) (type default)) (layer "Edge.Cuts"))
 (segment (start 21.204522 4.6) (end 20.304522 5.5) (width 0.6) (layer "F.Cu") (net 19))
 (segment (start 20.304522 6.504522) (end 21.6 7.8) (width 0.8) (layer "F.Cu") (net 19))
 (segment (start 20.304522 5.5) (end 20.304522 6.504522) (width 0.8) (layer "F.Cu") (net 19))
 (segment (start 22.2 4.6) (end 21.204522 4.6) (width 1) (layer "F.Cu") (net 19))
 (via (at 22.2 4.6) (size 0.6) (drill 0.3) (layers "F.Cu" "B.Cu") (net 19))
 (via (at 21.6 7.8) (size 0.6) (drill 0.3) (layers "F.Cu" "B.Cu") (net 19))
 (segment (start 22.054522 11.345478) (end 22.054522 12.05) (width 0.6) (layer "B.Cu") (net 19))
 (segment (start 21.6 7.8) (end 22.4 8.6) (width 0.8) (layer "B.Cu") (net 19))
 (segment (start 23.3 1.6) (end 24.2 2.5) (width 0.8) (layer "B.Cu") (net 19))
 (segment (start 22.4 8.6) (end 22.4 11) (width 0.8) (layer "B.Cu") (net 19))
 (segment (start 22.6 5.8) (end 22.2 5.4) (width 1) (layer "B.Cu") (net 19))
 (segment (start 22.4 11) (end 22.054522 11.345478) (width 0.8) (layer "B.Cu") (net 19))
 (segment (start 24.2 5.6) (end 24 5.8) (width 1) (layer "B.Cu") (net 19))
 (segment (start 24 5.8) (end 22.6 5.8) (width 1) (layer "B.Cu") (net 19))
 (segment (start 24.2 4.6) (end 24.2 5.6) (width 1) (layer "B.Cu") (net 19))
 (segment (start 24.2 2.5) (end 24.2 4.6) (width 1) (layer "B.Cu") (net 19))
 (segment (start 22.2 5.4) (end 22.2 4.6) (width 1) (layer "B.Cu") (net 19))
 (segment (start 22.054522 16.317022) (end 22.3375 16.6) (width 0.8) (layer "B.Cu") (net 4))
 (segment (start 11.2875 30.85) (end 11.4 30.7375) (width 0.8) (layer "B.Cu") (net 4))
 (segment (start 9.35 30.85) (end 11.2875 30.85) (width 0.8) (layer "B.Cu") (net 4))
 (segment (start 22.054522 14.75) (end 22.054522 16.317022) (width 0.8) (layer "B.Cu") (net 4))
 (segment (start 7.8 23) (end 9.7 23) (width 0.8) (layer "F.Cu") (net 18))
 (segment (start 9.7 23) (end 10.6 23.9) (width 1) (layer "F.Cu") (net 18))
 (segment (start 7.4 23.4) (end 7.8 23) (width 0.8) (layer "F.Cu") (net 18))
 (segment (start 10.6 23.9) (end 10.6 24.6) (width 1) (layer "F.Cu") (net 18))
 (via (at 7.4 23.4) (size 0.6) (drill 0.3) (layers "F.Cu" "B.Cu") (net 18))
 (via (at 10.6 24.6) (size 0.6) (drill 0.3) (layers "F.Cu" "B.Cu") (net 18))
 (segment (start 8.8 25.2) (end 8.8 28.055635) (width 1) (layer "B.Cu") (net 18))
 (segment (start 6.65 30.85) (end 7.4 30.1) (width 0.8) (layer "B.Cu") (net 18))
 (segment (start 7.4 30.1) (end 7.4 23.4) (width 0.8) (layer "B.Cu") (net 18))
 (segment (start 10.6 24.6) (end 10 25.2) (width 1) (layer "B.Cu") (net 18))
 (segment (start 10 25.2) (end 8.8 25.2) (width 1) (layer "B.Cu") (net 18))
 (segment (start 9.3 28.4) (end 9.144365 28.4) (width 0.6) (layer "B.Cu") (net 18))
 (segment (start 8.8 28.055635) (end 8.85 28.105635) (width 1) (layer "B.Cu") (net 18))
 (segment (start 9.144365 28.4) (end 8.8 28.055635) (width 0.6) (layer "B.Cu") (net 18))
 (segment (start 20.154522 12.829999) (end 20.924523 13.6) (width 0.2) (layer "B.Cu") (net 22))
 (segment (start 20.924523 13.6) (end 24 13.6) (width 0.2) (layer "B.Cu") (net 22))
 (segment (start 24 13.6) (end 24.9 14.5) (width 0.2) (layer "B.Cu") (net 22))
 (segment (start 24.9 14.5) (end 24.9 17.066722) (width 0.2) (layer "B.Cu") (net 22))
 (segment (start 20.154522 12.05) (end 20.154522 12.829999) (width 0.2) (layer "B.Cu") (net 22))
 (segment (start 23.708654 18) (end 22.84 18.868654) (width 0.2) (layer "B.Cu") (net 22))
 (segment (start 22.84 20.535) (end 22.84 18.727233) (width 0.2) (layer "B.Cu") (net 22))
 (segment (start 23.966722 18) (end 23.708654 18) (width 0.2) (layer "B.Cu") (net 22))
 (segment (start 22.84 18.868654) (end 22.84 19.8) (width 0.2) (layer "B.Cu") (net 22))
 (segment (start 24.9 17.066722) (end 23.966722 18) (width 0.2) (layer "B.Cu") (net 22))
 (segment (start 24.09 21.785) (end 22.84 20.535) (width 0.2) (layer "B.Cu") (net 22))
 (segment (start 22.134314 20.395) (end 20.595 20.395) (width 0.2) (layer "B.Cu") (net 20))
 (segment (start 20.154522 19.954522) (end 20.154522 14.75) (width 0.2) (layer "B.Cu") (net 20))
 (segment (start 22.94 23.175) (end 22.94 21.200686) (width 0.2) (layer "B.Cu") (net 20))
 (segment (start 24.09 24.325) (end 22.94 23.175) (width 0.2) (layer "B.Cu") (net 20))
 (segment (start 20.595 20.395) (end 20.154522 19.954522) (width 0.2) (layer "B.Cu") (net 20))
 (segment (start 22.94 21.200686) (end 22.134314 20.395) (width 0.2) (layer "B.Cu") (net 20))
 (segment (start 21.4 30) (end 19.775 31.625) (width 0.2) (layer "B.Cu") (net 21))
 (segment (start 10.933278 31.625) (end 10.4 32.158278) (width 0.2) (layer "B.Cu") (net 21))
 (segment (start 21.4 24.475) (end 21.4 30) (width 0.2) (layer "B.Cu") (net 21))
 (segment (start 9.85 32.75) (end 9.35 32.75) (width 0.2) (layer "B.Cu") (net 21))
 (segment (start 19.775 31.625) (end 10.933278 31.625) (width 0.2) (layer "B.Cu") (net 21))
 (segment (start 10.4 32.2) (end 9.85 32.75) (width 0.2) (layer "B.Cu") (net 21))
 (segment (start 10.4 32.158278) (end 10.4 32.2) (width 0.2) (layer "B.Cu") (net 21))
 (segment (start 21.55 24.325) (end 21.4 24.475) (width 0.2) (layer "B.Cu") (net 21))
 (segment (start 20.2 23.135) (end 21.55 21.785) (width 0.2) (layer "B.Cu") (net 23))
 (segment (start 20.8 29.2) (end 20.8 26) (width 0.2) (layer "B.Cu") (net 23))
 (segment (start 8.9 29.9) (end 20.1 29.9) (width 0.2) (layer "B.Cu") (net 23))
 (segment (start 6.65 32.75) (end 7.429999 32.75) (width 0.2) (layer "B.Cu") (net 23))
 (segment (start 7.429999 32.75) (end 8.27 31.909999) (width 0.2) (layer "B.Cu") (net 23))
 (segment (start 20.1 29.9) (end 20.8 29.2) (width 0.2) (layer "B.Cu") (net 23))
 (segment (start 20.2 25.4) (end 20.2 23.135) (width 0.2) (layer "B.Cu") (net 23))
 (segment (start 8.6 30) (end 8.8 30) (width 0.2) (layer "B.Cu") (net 23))
 (segment (start 8.27 30.33) (end 8.6 30) (width 0.2) (layer "B.Cu") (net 23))
 (segment (start 8.27 31.909999) (end 8.27 30.33) (width 0.2) (layer "B.Cu") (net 23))
 (segment (start 8.8 30) (end 8.9 29.9) (width 0.2) (layer "B.Cu") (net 23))
 (segment (start 20.8 26) (end 20.2 25.4) (width 0.2) (layer "B.Cu") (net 23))
 (segment (start 21.104522 10.3125) (end 21.217022 10.2) (width 0.5) (layer "B.Cu") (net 31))
 (segment (start 21.104522 12.05) (end 21.104522 10.3125) (width 0.5) (layer "B.Cu") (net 31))
 (segment (start 5.1125 31.8) (end 4.7625 32.15) (width 0.6) (layer "B.Cu") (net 26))
 (segment (start 5.1125 31.8) (end 6.65 31.8) (width 0.6) (layer "B.Cu") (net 26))
 (segment (start 4.7625 32.15) (end 4.7625 32.65) (width 0.6) (layer "B.Cu") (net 26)))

